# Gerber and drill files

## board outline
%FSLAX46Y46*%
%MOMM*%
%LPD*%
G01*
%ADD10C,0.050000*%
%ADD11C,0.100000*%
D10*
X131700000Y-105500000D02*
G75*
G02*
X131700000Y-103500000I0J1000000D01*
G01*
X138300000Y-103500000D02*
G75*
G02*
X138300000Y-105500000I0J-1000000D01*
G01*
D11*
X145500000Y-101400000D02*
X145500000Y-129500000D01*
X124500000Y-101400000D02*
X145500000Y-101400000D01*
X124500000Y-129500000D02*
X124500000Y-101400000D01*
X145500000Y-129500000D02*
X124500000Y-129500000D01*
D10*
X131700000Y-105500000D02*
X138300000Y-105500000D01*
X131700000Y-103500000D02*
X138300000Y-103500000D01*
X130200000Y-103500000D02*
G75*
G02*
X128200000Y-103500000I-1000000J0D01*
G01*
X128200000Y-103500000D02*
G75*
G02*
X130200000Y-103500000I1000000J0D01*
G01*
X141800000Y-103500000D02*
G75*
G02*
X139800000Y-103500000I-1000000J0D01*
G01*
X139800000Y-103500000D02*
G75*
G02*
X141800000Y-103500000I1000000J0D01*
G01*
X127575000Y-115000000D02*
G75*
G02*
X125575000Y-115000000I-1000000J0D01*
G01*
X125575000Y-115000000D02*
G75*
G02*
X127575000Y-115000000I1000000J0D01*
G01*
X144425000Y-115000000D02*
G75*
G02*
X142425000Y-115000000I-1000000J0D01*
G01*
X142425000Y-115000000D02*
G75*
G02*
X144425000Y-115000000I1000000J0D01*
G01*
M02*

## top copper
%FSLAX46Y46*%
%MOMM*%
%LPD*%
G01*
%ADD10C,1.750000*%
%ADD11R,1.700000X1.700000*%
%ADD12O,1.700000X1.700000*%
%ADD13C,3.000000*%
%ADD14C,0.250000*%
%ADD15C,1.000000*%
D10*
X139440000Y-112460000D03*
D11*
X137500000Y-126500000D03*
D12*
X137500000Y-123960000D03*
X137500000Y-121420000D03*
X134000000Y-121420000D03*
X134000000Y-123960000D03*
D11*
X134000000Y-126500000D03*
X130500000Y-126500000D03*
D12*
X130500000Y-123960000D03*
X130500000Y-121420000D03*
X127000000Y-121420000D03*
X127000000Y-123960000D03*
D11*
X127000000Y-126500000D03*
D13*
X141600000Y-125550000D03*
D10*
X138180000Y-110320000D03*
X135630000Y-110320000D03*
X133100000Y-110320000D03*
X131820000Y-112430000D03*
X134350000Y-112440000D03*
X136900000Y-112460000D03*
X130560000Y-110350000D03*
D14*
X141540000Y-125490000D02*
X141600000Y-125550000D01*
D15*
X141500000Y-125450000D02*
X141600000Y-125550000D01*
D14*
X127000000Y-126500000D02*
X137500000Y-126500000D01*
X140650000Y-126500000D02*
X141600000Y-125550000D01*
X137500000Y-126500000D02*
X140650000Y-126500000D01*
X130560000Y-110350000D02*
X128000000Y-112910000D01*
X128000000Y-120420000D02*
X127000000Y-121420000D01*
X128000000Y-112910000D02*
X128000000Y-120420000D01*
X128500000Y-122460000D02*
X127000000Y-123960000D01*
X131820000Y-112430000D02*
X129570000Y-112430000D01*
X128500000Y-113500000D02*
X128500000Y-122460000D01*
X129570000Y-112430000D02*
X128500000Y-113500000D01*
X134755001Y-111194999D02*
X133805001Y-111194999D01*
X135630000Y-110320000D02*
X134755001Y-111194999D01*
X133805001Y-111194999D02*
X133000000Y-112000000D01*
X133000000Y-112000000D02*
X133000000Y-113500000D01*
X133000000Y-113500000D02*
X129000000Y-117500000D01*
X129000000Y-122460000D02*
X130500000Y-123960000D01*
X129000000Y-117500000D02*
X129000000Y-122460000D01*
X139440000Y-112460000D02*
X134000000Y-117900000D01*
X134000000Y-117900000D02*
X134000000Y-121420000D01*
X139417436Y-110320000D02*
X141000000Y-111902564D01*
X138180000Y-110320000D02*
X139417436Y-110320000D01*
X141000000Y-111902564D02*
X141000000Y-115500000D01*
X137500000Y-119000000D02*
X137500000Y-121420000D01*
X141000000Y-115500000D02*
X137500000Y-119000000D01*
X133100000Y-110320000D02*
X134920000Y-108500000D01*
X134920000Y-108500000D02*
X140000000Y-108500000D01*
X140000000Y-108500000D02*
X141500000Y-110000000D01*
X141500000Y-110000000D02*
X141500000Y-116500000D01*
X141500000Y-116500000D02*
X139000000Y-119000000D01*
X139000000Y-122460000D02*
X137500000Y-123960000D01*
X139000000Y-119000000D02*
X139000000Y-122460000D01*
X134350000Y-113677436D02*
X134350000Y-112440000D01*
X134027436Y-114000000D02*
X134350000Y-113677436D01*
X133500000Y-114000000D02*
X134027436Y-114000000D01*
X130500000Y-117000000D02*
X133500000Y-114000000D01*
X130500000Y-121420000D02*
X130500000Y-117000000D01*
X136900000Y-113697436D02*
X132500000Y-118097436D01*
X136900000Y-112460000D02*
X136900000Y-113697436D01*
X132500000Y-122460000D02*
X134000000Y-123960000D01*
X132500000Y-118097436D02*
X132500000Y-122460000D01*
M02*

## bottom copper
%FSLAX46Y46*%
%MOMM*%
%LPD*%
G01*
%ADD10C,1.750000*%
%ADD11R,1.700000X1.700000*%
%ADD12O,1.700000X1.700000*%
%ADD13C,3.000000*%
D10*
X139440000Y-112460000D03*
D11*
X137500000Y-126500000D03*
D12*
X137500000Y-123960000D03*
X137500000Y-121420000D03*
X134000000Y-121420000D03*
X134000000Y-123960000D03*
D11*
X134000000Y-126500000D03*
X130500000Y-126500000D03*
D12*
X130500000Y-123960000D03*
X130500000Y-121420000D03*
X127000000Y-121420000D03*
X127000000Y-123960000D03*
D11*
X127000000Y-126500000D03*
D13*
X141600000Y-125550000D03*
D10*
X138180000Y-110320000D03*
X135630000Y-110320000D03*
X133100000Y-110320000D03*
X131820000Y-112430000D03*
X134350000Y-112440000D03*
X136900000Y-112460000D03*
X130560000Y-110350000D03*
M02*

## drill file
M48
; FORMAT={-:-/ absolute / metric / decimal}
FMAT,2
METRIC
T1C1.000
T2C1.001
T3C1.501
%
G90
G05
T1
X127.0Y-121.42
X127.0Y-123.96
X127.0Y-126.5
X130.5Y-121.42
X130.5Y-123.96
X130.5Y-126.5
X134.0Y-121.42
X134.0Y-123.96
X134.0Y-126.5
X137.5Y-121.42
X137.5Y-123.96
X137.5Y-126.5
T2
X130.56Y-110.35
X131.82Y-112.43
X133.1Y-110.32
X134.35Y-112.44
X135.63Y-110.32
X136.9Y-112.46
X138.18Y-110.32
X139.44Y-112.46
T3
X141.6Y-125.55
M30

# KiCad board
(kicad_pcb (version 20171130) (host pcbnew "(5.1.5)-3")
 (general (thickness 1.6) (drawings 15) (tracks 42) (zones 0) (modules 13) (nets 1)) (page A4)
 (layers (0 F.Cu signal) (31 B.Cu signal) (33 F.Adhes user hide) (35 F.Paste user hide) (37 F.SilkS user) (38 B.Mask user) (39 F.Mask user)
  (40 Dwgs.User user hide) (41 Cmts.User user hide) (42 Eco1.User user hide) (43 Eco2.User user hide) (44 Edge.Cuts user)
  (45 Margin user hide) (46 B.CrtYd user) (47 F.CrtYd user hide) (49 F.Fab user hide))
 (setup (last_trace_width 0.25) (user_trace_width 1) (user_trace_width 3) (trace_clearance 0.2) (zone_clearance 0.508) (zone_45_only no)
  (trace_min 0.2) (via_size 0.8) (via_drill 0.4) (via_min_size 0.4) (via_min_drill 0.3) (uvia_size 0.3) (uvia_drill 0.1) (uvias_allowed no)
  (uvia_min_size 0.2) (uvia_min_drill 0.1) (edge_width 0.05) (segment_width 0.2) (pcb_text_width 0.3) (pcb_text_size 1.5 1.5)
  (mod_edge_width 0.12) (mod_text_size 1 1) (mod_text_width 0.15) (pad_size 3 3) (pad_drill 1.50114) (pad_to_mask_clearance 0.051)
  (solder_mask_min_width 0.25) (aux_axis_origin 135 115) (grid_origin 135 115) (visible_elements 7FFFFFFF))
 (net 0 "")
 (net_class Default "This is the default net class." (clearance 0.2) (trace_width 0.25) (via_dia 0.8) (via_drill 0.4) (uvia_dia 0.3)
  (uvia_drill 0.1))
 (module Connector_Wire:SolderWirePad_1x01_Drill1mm (layer F.Cu) (at 139.44 112.46)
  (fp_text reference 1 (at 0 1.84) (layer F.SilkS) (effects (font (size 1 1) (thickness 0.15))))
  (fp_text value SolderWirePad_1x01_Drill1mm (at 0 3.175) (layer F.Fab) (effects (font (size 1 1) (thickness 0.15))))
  (pad 1 thru_hole circle (at 0 0) (size 1.75 1.75) (drill 1.00076) (layers *.Cu *.Mask)))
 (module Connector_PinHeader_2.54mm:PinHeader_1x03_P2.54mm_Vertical (layer F.Cu) (at 137.5 126.5 180)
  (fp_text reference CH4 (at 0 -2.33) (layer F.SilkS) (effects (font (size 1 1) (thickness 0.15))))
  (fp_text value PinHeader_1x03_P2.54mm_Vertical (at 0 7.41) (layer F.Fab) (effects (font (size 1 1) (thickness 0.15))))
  (pad 1 thru_hole rect (at 0 0 180) (size 1.7 1.7) (drill 1) (layers *.Cu *.Mask))
  (pad 2 thru_hole oval (at 0 2.54 180) (size 1.7 1.7) (drill 1) (layers *.Cu *.Mask))
  (pad 3 thru_hole oval (at 0 5.08 180) (size 1.7 1.7) (drill 1) (layers *.Cu *.Mask)))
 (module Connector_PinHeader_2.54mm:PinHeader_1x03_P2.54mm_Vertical (layer F.Cu) (at 134 126.5 180)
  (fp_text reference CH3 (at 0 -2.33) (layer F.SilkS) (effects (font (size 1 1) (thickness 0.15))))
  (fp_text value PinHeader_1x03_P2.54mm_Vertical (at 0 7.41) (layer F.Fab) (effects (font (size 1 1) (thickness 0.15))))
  (pad 3 thru_hole oval (at 0 5.08 180) (size 1.7 1.7) (drill 1) (layers *.Cu *.Mask))
  (pad 2 thru_hole oval (at 0 2.54 180) (size 1.7 1.7) (drill 1) (layers *.Cu *.Mask))
  (pad 1 thru_hole rect (at 0 0 180) (size 1.7 1.7) (drill 1) (layers *.Cu *.Mask)))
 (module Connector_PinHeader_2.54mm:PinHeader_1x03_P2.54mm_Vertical (layer F.Cu) (at 130.5 126.5 180)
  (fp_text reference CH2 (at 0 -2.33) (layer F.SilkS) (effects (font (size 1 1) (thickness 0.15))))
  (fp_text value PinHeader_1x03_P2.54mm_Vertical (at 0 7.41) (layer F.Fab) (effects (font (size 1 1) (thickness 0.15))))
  (pad 1 thru_hole rect (at 0 0 180) (size 1.7 1.7) (drill 1) (layers *.Cu *.Mask))
  (pad 2 thru_hole oval (at 0 2.54 180) (size 1.7 1.7) (drill 1) (layers *.Cu *.Mask))
  (pad 3 thru_hole oval (at 0 5.08 180) (size 1.7 1.7) (drill 1) (layers *.Cu *.Mask)))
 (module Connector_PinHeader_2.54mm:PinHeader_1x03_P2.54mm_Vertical (layer F.Cu) (at 127 126.5 180)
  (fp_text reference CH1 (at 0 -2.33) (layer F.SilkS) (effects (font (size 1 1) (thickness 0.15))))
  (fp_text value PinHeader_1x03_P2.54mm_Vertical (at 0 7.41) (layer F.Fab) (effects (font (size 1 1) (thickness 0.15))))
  (pad 3 thru_hole oval (at 0 5.08 180) (size 1.7 1.7) (drill 1) (layers *.Cu *.Mask))
  (pad 2 thru_hole oval (at 0 2.54 180) (size 1.7 1.7) (drill 1) (layers *.Cu *.Mask))
  (pad 1 thru_hole rect (at 0 0 180) (size 1.7 1.7) (drill 1) (layers *.Cu *.Mask)))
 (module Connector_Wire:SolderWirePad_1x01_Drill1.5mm (layer F.Cu) (at 141.6 125.55)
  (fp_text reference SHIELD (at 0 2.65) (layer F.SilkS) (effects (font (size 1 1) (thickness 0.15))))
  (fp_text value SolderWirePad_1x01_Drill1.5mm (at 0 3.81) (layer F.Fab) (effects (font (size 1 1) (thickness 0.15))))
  (pad 1 thru_hole circle (at 0 0) (size 3 3) (drill 1.50114) (layers *.Cu *.Mask)))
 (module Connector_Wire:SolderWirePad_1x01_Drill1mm (layer F.Cu) (at 138.18 110.32)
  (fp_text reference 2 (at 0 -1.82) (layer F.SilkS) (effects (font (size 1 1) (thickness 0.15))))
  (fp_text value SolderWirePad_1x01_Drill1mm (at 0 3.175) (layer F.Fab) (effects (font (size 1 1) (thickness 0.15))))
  (pad 1 thru_hole circle (at 0 0) (size 1.75 1.75) (drill 1.00076) (layers *.Cu *.Mask)))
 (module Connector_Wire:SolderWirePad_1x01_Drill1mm (layer F.Cu) (at 135.63 110.32)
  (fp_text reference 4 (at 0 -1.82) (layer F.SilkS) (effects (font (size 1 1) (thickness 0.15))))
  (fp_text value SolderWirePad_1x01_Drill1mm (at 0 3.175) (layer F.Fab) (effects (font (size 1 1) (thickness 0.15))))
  (pad 1 thru_hole circle (at 0 0) (size 1.75 1.75) (drill 1.00076) (layers *.Cu *.Mask)))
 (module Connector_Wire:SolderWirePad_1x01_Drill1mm (layer F.Cu) (at 133.1 110.32)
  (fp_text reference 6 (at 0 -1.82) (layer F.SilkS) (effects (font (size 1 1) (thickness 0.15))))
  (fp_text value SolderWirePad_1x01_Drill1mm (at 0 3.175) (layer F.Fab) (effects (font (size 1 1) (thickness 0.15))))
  (pad 1 thru_hole circle (at 0 0) (size 1.75 1.75) (drill 1.00076) (layers *.Cu *.Mask)))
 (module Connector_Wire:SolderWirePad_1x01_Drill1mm (layer F.Cu) (at 131.82 112.43)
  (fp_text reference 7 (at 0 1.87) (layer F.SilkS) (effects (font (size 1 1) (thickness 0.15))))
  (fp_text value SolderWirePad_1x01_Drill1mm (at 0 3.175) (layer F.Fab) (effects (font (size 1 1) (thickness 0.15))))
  (pad 1 thru_hole circle (at 0 0) (size 1.75 1.75) (drill 1.00076) (layers *.Cu *.Mask)))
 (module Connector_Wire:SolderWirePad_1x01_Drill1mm (layer F.Cu) (at 134.35 112.44)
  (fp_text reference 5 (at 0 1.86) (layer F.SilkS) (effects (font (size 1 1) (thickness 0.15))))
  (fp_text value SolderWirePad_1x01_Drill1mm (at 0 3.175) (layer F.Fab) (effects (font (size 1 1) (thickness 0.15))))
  (pad 1 thru_hole circle (at 0 0) (size 1.75 1.75) (drill 1.00076) (layers *.Cu *.Mask)))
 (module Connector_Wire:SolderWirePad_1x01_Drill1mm (layer F.Cu) (at 136.9 112.46)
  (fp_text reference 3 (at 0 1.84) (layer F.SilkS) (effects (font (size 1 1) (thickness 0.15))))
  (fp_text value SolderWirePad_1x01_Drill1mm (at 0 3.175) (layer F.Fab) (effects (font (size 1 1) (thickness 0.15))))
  (pad 1 thru_hole circle (at 0 0) (size 1.75 1.75) (drill 1.00076) (layers *.Cu *.Mask)))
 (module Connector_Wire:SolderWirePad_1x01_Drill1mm (layer F.Cu) (at 130.56 110.35)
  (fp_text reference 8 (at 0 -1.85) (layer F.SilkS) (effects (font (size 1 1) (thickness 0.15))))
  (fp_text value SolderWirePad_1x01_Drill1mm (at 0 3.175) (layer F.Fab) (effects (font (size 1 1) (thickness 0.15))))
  (pad 1 thru_hole circle (at 0 0) (size 1.75 1.75) (drill 1.00076) (layers *.Cu *.Mask)))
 (gr_arc (start 131.7 104.5) (end 131.7 103.5) (angle -180) (layer Edge.Cuts) (width 0.05))
 (gr_arc (start 138.3 104.5) (end 138.3 105.5) (angle -180) (layer Edge.Cuts) (width 0.05))
 (gr_line (start 145.5 101.4) (end 145.5 129.5) (layer Edge.Cuts) (width 0.1))
 (gr_line (start 124.5 101.4) (end 145.5 101.4) (layer Edge.Cuts) (width 0.1))
 (gr_line (start 124.5 129.5) (end 124.5 101.4) (layer Edge.Cuts) (width 0.1))
 (gr_line (start 145.5 129.5) (end 124.5 129.5) (layer Edge.Cuts) (width 0.1))
 (gr_line (start 131.7 105.5) (end 138.3 105.5) (layer Edge.Cuts) (width 0.05))
 (gr_line (start 131.7 103.5) (end 138.3 103.5) (layer Edge.Cuts) (width 0.05))
 (gr_circle (center 129.2 103.5) (end 130.2 103.5) (layer Edge.Cuts) (width 0.05))
 (gr_circle (center 140.8 103.5) (end 141.8 103.5) (layer Edge.Cuts) (width 0.05))
 (gr_circle (center 126.575 115) (end 127.575 115) (layer Edge.Cuts) (width 0.05))
 (gr_circle (center 143.425 115) (end 144.425 115) (layer Edge.Cuts) (width 0.05))
 (segment (start 141.54 125.49) (end 141.6 125.55) (width 0.25) (layer F.Cu) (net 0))
 (segment (start 141.5 125.45) (end 141.6 125.55) (width 1) (layer F.Cu) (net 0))
 (segment (start 127 126.5) (end 137.5 126.5) (width 0.25) (layer F.Cu) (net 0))
 (segment (start 140.65 126.5) (end 141.6 125.55) (width 0.25) (layer F.Cu) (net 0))
 (segment (start 137.5 126.5) (end 140.65 126.5) (width 0.25) (layer F.Cu) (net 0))
 (segment (start 130.56 110.35) (end 128 112.91) (width 0.25) (layer F.Cu) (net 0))
 (segment (start 128 120.42) (end 127 121.42) (width 0.25) (layer F.Cu) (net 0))
 (segment (start 128 112.91) (end 128 120.42) (width 0.25) (layer F.Cu) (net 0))
 (segment (start 128.5 122.46) (end 127 123.96) (width 0.25) (layer F.Cu) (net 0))
 (segment (start 131.82 112.43) (end 129.57 112.43) (width 0.25) (layer F.Cu) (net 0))
 (segment (start 128.5 113.5) (end 128.5 122.46) (width 0.25) (layer F.Cu) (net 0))
 (segment (start 129.57 112.43) (end 128.5 113.5) (width 0.25) (layer F.Cu) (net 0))
 (segment (start 134.755001 111.194999) (end 133.805001 111.194999) (width 0.25) (layer F.Cu) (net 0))
 (segment (start 135.63 110.32) (end 134.755001 111.194999) (width 0.25) (layer F.Cu) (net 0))
 (segment (start 133.805001 111.194999) (end 133 112) (width 0.25) (layer F.Cu) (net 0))
 (segment (start 133 112) (end 133 113.5) (width 0.25) (layer F.Cu) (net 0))
 (segment (start 133 113.5) (end 129 117.5) (width 0.25) (layer F.Cu) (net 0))
 (segment (start 129 122.46) (end 130.5 123.96) (width 0.25) (layer F.Cu) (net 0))
 (segment (start 129 117.5) (end 129 122.46) (width 0.25) (layer F.Cu) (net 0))
 (segment (start 139.44 112.46) (end 134 117.9) (width 0.25) (layer F.Cu) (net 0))
 (segment (start 134 117.9) (end 134 121.42) (width 0.25) (layer F.Cu) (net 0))
 (segment (start 139.417436 110.32) (end 141 111.902564) (width 0.25) (layer F.Cu) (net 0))
 (segment (start 138.18 110.32) (end 139.417436 110.32) (width 0.25) (layer F.Cu) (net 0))
 (segment (start 141 111.902564) (end 141 115.5) (width 0.25) (layer F.Cu) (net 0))
 (segment (start 137.5 119) (end 137.5 121.42) (width 0.25) (layer F.Cu) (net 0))
 (segment (start 141 115.5) (end 137.5 119) (width 0.25) (layer F.Cu) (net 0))
 (segment (start 133.1 110.32) (end 134.92 108.5) (width 0.25) (layer F.Cu) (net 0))
 (segment (start 134.92 108.5) (end 140 108.5) (width 0.25) (layer F.Cu) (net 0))
 (segment (start 140 108.5) (end 141.5 110) (width 0.25) (layer F.Cu) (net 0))
 (segment (start 141.5 110) (end 141.5 116.5) (width 0.25) (layer F.Cu) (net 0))
 (segment (start 141.5 116.5) (end 139 119) (width 0.25) (layer F.Cu) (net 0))
 (segment (start 139 122.46) (end 137.5 123.96) (width 0.25) (layer F.Cu) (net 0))
 (segment (start 139 119) (end 139 122.46) (width 0.25) (layer F.Cu) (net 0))
 (segment (start 134.35 113.677436) (end 134.35 112.44) (width 0.25) (layer F.Cu) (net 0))
 (segment (start 134.027436 114) (end 134.35 113.677436) (width 0.25) (layer F.Cu) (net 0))
 (segment (start 133.5 114) (end 134.027436 114) (width 0.25) (layer F.Cu) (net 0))
 (segment (start 130.5 117) (end 133.5 114) (width 0.25) (layer F.Cu) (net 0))
 (segment (start 130.5 121.42) (end 130.5 117) (width 0.25) (layer F.Cu) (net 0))
 (segment (start 136.9 113.697436) (end 132.5 118.097436) (width 0.25) (layer F.Cu) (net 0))
 (segment (start 136.9 112.46) (end 136.9 113.697436) (width 0.25) (layer F.Cu) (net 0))
 (segment (start 132.5 122.46) (end 134 123.96) (width 0.25) (layer F.Cu) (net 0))
 (segment (start 132.5 118.097436) (end 132.5 122.46) (width 0.25) (layer F.Cu) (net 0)))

